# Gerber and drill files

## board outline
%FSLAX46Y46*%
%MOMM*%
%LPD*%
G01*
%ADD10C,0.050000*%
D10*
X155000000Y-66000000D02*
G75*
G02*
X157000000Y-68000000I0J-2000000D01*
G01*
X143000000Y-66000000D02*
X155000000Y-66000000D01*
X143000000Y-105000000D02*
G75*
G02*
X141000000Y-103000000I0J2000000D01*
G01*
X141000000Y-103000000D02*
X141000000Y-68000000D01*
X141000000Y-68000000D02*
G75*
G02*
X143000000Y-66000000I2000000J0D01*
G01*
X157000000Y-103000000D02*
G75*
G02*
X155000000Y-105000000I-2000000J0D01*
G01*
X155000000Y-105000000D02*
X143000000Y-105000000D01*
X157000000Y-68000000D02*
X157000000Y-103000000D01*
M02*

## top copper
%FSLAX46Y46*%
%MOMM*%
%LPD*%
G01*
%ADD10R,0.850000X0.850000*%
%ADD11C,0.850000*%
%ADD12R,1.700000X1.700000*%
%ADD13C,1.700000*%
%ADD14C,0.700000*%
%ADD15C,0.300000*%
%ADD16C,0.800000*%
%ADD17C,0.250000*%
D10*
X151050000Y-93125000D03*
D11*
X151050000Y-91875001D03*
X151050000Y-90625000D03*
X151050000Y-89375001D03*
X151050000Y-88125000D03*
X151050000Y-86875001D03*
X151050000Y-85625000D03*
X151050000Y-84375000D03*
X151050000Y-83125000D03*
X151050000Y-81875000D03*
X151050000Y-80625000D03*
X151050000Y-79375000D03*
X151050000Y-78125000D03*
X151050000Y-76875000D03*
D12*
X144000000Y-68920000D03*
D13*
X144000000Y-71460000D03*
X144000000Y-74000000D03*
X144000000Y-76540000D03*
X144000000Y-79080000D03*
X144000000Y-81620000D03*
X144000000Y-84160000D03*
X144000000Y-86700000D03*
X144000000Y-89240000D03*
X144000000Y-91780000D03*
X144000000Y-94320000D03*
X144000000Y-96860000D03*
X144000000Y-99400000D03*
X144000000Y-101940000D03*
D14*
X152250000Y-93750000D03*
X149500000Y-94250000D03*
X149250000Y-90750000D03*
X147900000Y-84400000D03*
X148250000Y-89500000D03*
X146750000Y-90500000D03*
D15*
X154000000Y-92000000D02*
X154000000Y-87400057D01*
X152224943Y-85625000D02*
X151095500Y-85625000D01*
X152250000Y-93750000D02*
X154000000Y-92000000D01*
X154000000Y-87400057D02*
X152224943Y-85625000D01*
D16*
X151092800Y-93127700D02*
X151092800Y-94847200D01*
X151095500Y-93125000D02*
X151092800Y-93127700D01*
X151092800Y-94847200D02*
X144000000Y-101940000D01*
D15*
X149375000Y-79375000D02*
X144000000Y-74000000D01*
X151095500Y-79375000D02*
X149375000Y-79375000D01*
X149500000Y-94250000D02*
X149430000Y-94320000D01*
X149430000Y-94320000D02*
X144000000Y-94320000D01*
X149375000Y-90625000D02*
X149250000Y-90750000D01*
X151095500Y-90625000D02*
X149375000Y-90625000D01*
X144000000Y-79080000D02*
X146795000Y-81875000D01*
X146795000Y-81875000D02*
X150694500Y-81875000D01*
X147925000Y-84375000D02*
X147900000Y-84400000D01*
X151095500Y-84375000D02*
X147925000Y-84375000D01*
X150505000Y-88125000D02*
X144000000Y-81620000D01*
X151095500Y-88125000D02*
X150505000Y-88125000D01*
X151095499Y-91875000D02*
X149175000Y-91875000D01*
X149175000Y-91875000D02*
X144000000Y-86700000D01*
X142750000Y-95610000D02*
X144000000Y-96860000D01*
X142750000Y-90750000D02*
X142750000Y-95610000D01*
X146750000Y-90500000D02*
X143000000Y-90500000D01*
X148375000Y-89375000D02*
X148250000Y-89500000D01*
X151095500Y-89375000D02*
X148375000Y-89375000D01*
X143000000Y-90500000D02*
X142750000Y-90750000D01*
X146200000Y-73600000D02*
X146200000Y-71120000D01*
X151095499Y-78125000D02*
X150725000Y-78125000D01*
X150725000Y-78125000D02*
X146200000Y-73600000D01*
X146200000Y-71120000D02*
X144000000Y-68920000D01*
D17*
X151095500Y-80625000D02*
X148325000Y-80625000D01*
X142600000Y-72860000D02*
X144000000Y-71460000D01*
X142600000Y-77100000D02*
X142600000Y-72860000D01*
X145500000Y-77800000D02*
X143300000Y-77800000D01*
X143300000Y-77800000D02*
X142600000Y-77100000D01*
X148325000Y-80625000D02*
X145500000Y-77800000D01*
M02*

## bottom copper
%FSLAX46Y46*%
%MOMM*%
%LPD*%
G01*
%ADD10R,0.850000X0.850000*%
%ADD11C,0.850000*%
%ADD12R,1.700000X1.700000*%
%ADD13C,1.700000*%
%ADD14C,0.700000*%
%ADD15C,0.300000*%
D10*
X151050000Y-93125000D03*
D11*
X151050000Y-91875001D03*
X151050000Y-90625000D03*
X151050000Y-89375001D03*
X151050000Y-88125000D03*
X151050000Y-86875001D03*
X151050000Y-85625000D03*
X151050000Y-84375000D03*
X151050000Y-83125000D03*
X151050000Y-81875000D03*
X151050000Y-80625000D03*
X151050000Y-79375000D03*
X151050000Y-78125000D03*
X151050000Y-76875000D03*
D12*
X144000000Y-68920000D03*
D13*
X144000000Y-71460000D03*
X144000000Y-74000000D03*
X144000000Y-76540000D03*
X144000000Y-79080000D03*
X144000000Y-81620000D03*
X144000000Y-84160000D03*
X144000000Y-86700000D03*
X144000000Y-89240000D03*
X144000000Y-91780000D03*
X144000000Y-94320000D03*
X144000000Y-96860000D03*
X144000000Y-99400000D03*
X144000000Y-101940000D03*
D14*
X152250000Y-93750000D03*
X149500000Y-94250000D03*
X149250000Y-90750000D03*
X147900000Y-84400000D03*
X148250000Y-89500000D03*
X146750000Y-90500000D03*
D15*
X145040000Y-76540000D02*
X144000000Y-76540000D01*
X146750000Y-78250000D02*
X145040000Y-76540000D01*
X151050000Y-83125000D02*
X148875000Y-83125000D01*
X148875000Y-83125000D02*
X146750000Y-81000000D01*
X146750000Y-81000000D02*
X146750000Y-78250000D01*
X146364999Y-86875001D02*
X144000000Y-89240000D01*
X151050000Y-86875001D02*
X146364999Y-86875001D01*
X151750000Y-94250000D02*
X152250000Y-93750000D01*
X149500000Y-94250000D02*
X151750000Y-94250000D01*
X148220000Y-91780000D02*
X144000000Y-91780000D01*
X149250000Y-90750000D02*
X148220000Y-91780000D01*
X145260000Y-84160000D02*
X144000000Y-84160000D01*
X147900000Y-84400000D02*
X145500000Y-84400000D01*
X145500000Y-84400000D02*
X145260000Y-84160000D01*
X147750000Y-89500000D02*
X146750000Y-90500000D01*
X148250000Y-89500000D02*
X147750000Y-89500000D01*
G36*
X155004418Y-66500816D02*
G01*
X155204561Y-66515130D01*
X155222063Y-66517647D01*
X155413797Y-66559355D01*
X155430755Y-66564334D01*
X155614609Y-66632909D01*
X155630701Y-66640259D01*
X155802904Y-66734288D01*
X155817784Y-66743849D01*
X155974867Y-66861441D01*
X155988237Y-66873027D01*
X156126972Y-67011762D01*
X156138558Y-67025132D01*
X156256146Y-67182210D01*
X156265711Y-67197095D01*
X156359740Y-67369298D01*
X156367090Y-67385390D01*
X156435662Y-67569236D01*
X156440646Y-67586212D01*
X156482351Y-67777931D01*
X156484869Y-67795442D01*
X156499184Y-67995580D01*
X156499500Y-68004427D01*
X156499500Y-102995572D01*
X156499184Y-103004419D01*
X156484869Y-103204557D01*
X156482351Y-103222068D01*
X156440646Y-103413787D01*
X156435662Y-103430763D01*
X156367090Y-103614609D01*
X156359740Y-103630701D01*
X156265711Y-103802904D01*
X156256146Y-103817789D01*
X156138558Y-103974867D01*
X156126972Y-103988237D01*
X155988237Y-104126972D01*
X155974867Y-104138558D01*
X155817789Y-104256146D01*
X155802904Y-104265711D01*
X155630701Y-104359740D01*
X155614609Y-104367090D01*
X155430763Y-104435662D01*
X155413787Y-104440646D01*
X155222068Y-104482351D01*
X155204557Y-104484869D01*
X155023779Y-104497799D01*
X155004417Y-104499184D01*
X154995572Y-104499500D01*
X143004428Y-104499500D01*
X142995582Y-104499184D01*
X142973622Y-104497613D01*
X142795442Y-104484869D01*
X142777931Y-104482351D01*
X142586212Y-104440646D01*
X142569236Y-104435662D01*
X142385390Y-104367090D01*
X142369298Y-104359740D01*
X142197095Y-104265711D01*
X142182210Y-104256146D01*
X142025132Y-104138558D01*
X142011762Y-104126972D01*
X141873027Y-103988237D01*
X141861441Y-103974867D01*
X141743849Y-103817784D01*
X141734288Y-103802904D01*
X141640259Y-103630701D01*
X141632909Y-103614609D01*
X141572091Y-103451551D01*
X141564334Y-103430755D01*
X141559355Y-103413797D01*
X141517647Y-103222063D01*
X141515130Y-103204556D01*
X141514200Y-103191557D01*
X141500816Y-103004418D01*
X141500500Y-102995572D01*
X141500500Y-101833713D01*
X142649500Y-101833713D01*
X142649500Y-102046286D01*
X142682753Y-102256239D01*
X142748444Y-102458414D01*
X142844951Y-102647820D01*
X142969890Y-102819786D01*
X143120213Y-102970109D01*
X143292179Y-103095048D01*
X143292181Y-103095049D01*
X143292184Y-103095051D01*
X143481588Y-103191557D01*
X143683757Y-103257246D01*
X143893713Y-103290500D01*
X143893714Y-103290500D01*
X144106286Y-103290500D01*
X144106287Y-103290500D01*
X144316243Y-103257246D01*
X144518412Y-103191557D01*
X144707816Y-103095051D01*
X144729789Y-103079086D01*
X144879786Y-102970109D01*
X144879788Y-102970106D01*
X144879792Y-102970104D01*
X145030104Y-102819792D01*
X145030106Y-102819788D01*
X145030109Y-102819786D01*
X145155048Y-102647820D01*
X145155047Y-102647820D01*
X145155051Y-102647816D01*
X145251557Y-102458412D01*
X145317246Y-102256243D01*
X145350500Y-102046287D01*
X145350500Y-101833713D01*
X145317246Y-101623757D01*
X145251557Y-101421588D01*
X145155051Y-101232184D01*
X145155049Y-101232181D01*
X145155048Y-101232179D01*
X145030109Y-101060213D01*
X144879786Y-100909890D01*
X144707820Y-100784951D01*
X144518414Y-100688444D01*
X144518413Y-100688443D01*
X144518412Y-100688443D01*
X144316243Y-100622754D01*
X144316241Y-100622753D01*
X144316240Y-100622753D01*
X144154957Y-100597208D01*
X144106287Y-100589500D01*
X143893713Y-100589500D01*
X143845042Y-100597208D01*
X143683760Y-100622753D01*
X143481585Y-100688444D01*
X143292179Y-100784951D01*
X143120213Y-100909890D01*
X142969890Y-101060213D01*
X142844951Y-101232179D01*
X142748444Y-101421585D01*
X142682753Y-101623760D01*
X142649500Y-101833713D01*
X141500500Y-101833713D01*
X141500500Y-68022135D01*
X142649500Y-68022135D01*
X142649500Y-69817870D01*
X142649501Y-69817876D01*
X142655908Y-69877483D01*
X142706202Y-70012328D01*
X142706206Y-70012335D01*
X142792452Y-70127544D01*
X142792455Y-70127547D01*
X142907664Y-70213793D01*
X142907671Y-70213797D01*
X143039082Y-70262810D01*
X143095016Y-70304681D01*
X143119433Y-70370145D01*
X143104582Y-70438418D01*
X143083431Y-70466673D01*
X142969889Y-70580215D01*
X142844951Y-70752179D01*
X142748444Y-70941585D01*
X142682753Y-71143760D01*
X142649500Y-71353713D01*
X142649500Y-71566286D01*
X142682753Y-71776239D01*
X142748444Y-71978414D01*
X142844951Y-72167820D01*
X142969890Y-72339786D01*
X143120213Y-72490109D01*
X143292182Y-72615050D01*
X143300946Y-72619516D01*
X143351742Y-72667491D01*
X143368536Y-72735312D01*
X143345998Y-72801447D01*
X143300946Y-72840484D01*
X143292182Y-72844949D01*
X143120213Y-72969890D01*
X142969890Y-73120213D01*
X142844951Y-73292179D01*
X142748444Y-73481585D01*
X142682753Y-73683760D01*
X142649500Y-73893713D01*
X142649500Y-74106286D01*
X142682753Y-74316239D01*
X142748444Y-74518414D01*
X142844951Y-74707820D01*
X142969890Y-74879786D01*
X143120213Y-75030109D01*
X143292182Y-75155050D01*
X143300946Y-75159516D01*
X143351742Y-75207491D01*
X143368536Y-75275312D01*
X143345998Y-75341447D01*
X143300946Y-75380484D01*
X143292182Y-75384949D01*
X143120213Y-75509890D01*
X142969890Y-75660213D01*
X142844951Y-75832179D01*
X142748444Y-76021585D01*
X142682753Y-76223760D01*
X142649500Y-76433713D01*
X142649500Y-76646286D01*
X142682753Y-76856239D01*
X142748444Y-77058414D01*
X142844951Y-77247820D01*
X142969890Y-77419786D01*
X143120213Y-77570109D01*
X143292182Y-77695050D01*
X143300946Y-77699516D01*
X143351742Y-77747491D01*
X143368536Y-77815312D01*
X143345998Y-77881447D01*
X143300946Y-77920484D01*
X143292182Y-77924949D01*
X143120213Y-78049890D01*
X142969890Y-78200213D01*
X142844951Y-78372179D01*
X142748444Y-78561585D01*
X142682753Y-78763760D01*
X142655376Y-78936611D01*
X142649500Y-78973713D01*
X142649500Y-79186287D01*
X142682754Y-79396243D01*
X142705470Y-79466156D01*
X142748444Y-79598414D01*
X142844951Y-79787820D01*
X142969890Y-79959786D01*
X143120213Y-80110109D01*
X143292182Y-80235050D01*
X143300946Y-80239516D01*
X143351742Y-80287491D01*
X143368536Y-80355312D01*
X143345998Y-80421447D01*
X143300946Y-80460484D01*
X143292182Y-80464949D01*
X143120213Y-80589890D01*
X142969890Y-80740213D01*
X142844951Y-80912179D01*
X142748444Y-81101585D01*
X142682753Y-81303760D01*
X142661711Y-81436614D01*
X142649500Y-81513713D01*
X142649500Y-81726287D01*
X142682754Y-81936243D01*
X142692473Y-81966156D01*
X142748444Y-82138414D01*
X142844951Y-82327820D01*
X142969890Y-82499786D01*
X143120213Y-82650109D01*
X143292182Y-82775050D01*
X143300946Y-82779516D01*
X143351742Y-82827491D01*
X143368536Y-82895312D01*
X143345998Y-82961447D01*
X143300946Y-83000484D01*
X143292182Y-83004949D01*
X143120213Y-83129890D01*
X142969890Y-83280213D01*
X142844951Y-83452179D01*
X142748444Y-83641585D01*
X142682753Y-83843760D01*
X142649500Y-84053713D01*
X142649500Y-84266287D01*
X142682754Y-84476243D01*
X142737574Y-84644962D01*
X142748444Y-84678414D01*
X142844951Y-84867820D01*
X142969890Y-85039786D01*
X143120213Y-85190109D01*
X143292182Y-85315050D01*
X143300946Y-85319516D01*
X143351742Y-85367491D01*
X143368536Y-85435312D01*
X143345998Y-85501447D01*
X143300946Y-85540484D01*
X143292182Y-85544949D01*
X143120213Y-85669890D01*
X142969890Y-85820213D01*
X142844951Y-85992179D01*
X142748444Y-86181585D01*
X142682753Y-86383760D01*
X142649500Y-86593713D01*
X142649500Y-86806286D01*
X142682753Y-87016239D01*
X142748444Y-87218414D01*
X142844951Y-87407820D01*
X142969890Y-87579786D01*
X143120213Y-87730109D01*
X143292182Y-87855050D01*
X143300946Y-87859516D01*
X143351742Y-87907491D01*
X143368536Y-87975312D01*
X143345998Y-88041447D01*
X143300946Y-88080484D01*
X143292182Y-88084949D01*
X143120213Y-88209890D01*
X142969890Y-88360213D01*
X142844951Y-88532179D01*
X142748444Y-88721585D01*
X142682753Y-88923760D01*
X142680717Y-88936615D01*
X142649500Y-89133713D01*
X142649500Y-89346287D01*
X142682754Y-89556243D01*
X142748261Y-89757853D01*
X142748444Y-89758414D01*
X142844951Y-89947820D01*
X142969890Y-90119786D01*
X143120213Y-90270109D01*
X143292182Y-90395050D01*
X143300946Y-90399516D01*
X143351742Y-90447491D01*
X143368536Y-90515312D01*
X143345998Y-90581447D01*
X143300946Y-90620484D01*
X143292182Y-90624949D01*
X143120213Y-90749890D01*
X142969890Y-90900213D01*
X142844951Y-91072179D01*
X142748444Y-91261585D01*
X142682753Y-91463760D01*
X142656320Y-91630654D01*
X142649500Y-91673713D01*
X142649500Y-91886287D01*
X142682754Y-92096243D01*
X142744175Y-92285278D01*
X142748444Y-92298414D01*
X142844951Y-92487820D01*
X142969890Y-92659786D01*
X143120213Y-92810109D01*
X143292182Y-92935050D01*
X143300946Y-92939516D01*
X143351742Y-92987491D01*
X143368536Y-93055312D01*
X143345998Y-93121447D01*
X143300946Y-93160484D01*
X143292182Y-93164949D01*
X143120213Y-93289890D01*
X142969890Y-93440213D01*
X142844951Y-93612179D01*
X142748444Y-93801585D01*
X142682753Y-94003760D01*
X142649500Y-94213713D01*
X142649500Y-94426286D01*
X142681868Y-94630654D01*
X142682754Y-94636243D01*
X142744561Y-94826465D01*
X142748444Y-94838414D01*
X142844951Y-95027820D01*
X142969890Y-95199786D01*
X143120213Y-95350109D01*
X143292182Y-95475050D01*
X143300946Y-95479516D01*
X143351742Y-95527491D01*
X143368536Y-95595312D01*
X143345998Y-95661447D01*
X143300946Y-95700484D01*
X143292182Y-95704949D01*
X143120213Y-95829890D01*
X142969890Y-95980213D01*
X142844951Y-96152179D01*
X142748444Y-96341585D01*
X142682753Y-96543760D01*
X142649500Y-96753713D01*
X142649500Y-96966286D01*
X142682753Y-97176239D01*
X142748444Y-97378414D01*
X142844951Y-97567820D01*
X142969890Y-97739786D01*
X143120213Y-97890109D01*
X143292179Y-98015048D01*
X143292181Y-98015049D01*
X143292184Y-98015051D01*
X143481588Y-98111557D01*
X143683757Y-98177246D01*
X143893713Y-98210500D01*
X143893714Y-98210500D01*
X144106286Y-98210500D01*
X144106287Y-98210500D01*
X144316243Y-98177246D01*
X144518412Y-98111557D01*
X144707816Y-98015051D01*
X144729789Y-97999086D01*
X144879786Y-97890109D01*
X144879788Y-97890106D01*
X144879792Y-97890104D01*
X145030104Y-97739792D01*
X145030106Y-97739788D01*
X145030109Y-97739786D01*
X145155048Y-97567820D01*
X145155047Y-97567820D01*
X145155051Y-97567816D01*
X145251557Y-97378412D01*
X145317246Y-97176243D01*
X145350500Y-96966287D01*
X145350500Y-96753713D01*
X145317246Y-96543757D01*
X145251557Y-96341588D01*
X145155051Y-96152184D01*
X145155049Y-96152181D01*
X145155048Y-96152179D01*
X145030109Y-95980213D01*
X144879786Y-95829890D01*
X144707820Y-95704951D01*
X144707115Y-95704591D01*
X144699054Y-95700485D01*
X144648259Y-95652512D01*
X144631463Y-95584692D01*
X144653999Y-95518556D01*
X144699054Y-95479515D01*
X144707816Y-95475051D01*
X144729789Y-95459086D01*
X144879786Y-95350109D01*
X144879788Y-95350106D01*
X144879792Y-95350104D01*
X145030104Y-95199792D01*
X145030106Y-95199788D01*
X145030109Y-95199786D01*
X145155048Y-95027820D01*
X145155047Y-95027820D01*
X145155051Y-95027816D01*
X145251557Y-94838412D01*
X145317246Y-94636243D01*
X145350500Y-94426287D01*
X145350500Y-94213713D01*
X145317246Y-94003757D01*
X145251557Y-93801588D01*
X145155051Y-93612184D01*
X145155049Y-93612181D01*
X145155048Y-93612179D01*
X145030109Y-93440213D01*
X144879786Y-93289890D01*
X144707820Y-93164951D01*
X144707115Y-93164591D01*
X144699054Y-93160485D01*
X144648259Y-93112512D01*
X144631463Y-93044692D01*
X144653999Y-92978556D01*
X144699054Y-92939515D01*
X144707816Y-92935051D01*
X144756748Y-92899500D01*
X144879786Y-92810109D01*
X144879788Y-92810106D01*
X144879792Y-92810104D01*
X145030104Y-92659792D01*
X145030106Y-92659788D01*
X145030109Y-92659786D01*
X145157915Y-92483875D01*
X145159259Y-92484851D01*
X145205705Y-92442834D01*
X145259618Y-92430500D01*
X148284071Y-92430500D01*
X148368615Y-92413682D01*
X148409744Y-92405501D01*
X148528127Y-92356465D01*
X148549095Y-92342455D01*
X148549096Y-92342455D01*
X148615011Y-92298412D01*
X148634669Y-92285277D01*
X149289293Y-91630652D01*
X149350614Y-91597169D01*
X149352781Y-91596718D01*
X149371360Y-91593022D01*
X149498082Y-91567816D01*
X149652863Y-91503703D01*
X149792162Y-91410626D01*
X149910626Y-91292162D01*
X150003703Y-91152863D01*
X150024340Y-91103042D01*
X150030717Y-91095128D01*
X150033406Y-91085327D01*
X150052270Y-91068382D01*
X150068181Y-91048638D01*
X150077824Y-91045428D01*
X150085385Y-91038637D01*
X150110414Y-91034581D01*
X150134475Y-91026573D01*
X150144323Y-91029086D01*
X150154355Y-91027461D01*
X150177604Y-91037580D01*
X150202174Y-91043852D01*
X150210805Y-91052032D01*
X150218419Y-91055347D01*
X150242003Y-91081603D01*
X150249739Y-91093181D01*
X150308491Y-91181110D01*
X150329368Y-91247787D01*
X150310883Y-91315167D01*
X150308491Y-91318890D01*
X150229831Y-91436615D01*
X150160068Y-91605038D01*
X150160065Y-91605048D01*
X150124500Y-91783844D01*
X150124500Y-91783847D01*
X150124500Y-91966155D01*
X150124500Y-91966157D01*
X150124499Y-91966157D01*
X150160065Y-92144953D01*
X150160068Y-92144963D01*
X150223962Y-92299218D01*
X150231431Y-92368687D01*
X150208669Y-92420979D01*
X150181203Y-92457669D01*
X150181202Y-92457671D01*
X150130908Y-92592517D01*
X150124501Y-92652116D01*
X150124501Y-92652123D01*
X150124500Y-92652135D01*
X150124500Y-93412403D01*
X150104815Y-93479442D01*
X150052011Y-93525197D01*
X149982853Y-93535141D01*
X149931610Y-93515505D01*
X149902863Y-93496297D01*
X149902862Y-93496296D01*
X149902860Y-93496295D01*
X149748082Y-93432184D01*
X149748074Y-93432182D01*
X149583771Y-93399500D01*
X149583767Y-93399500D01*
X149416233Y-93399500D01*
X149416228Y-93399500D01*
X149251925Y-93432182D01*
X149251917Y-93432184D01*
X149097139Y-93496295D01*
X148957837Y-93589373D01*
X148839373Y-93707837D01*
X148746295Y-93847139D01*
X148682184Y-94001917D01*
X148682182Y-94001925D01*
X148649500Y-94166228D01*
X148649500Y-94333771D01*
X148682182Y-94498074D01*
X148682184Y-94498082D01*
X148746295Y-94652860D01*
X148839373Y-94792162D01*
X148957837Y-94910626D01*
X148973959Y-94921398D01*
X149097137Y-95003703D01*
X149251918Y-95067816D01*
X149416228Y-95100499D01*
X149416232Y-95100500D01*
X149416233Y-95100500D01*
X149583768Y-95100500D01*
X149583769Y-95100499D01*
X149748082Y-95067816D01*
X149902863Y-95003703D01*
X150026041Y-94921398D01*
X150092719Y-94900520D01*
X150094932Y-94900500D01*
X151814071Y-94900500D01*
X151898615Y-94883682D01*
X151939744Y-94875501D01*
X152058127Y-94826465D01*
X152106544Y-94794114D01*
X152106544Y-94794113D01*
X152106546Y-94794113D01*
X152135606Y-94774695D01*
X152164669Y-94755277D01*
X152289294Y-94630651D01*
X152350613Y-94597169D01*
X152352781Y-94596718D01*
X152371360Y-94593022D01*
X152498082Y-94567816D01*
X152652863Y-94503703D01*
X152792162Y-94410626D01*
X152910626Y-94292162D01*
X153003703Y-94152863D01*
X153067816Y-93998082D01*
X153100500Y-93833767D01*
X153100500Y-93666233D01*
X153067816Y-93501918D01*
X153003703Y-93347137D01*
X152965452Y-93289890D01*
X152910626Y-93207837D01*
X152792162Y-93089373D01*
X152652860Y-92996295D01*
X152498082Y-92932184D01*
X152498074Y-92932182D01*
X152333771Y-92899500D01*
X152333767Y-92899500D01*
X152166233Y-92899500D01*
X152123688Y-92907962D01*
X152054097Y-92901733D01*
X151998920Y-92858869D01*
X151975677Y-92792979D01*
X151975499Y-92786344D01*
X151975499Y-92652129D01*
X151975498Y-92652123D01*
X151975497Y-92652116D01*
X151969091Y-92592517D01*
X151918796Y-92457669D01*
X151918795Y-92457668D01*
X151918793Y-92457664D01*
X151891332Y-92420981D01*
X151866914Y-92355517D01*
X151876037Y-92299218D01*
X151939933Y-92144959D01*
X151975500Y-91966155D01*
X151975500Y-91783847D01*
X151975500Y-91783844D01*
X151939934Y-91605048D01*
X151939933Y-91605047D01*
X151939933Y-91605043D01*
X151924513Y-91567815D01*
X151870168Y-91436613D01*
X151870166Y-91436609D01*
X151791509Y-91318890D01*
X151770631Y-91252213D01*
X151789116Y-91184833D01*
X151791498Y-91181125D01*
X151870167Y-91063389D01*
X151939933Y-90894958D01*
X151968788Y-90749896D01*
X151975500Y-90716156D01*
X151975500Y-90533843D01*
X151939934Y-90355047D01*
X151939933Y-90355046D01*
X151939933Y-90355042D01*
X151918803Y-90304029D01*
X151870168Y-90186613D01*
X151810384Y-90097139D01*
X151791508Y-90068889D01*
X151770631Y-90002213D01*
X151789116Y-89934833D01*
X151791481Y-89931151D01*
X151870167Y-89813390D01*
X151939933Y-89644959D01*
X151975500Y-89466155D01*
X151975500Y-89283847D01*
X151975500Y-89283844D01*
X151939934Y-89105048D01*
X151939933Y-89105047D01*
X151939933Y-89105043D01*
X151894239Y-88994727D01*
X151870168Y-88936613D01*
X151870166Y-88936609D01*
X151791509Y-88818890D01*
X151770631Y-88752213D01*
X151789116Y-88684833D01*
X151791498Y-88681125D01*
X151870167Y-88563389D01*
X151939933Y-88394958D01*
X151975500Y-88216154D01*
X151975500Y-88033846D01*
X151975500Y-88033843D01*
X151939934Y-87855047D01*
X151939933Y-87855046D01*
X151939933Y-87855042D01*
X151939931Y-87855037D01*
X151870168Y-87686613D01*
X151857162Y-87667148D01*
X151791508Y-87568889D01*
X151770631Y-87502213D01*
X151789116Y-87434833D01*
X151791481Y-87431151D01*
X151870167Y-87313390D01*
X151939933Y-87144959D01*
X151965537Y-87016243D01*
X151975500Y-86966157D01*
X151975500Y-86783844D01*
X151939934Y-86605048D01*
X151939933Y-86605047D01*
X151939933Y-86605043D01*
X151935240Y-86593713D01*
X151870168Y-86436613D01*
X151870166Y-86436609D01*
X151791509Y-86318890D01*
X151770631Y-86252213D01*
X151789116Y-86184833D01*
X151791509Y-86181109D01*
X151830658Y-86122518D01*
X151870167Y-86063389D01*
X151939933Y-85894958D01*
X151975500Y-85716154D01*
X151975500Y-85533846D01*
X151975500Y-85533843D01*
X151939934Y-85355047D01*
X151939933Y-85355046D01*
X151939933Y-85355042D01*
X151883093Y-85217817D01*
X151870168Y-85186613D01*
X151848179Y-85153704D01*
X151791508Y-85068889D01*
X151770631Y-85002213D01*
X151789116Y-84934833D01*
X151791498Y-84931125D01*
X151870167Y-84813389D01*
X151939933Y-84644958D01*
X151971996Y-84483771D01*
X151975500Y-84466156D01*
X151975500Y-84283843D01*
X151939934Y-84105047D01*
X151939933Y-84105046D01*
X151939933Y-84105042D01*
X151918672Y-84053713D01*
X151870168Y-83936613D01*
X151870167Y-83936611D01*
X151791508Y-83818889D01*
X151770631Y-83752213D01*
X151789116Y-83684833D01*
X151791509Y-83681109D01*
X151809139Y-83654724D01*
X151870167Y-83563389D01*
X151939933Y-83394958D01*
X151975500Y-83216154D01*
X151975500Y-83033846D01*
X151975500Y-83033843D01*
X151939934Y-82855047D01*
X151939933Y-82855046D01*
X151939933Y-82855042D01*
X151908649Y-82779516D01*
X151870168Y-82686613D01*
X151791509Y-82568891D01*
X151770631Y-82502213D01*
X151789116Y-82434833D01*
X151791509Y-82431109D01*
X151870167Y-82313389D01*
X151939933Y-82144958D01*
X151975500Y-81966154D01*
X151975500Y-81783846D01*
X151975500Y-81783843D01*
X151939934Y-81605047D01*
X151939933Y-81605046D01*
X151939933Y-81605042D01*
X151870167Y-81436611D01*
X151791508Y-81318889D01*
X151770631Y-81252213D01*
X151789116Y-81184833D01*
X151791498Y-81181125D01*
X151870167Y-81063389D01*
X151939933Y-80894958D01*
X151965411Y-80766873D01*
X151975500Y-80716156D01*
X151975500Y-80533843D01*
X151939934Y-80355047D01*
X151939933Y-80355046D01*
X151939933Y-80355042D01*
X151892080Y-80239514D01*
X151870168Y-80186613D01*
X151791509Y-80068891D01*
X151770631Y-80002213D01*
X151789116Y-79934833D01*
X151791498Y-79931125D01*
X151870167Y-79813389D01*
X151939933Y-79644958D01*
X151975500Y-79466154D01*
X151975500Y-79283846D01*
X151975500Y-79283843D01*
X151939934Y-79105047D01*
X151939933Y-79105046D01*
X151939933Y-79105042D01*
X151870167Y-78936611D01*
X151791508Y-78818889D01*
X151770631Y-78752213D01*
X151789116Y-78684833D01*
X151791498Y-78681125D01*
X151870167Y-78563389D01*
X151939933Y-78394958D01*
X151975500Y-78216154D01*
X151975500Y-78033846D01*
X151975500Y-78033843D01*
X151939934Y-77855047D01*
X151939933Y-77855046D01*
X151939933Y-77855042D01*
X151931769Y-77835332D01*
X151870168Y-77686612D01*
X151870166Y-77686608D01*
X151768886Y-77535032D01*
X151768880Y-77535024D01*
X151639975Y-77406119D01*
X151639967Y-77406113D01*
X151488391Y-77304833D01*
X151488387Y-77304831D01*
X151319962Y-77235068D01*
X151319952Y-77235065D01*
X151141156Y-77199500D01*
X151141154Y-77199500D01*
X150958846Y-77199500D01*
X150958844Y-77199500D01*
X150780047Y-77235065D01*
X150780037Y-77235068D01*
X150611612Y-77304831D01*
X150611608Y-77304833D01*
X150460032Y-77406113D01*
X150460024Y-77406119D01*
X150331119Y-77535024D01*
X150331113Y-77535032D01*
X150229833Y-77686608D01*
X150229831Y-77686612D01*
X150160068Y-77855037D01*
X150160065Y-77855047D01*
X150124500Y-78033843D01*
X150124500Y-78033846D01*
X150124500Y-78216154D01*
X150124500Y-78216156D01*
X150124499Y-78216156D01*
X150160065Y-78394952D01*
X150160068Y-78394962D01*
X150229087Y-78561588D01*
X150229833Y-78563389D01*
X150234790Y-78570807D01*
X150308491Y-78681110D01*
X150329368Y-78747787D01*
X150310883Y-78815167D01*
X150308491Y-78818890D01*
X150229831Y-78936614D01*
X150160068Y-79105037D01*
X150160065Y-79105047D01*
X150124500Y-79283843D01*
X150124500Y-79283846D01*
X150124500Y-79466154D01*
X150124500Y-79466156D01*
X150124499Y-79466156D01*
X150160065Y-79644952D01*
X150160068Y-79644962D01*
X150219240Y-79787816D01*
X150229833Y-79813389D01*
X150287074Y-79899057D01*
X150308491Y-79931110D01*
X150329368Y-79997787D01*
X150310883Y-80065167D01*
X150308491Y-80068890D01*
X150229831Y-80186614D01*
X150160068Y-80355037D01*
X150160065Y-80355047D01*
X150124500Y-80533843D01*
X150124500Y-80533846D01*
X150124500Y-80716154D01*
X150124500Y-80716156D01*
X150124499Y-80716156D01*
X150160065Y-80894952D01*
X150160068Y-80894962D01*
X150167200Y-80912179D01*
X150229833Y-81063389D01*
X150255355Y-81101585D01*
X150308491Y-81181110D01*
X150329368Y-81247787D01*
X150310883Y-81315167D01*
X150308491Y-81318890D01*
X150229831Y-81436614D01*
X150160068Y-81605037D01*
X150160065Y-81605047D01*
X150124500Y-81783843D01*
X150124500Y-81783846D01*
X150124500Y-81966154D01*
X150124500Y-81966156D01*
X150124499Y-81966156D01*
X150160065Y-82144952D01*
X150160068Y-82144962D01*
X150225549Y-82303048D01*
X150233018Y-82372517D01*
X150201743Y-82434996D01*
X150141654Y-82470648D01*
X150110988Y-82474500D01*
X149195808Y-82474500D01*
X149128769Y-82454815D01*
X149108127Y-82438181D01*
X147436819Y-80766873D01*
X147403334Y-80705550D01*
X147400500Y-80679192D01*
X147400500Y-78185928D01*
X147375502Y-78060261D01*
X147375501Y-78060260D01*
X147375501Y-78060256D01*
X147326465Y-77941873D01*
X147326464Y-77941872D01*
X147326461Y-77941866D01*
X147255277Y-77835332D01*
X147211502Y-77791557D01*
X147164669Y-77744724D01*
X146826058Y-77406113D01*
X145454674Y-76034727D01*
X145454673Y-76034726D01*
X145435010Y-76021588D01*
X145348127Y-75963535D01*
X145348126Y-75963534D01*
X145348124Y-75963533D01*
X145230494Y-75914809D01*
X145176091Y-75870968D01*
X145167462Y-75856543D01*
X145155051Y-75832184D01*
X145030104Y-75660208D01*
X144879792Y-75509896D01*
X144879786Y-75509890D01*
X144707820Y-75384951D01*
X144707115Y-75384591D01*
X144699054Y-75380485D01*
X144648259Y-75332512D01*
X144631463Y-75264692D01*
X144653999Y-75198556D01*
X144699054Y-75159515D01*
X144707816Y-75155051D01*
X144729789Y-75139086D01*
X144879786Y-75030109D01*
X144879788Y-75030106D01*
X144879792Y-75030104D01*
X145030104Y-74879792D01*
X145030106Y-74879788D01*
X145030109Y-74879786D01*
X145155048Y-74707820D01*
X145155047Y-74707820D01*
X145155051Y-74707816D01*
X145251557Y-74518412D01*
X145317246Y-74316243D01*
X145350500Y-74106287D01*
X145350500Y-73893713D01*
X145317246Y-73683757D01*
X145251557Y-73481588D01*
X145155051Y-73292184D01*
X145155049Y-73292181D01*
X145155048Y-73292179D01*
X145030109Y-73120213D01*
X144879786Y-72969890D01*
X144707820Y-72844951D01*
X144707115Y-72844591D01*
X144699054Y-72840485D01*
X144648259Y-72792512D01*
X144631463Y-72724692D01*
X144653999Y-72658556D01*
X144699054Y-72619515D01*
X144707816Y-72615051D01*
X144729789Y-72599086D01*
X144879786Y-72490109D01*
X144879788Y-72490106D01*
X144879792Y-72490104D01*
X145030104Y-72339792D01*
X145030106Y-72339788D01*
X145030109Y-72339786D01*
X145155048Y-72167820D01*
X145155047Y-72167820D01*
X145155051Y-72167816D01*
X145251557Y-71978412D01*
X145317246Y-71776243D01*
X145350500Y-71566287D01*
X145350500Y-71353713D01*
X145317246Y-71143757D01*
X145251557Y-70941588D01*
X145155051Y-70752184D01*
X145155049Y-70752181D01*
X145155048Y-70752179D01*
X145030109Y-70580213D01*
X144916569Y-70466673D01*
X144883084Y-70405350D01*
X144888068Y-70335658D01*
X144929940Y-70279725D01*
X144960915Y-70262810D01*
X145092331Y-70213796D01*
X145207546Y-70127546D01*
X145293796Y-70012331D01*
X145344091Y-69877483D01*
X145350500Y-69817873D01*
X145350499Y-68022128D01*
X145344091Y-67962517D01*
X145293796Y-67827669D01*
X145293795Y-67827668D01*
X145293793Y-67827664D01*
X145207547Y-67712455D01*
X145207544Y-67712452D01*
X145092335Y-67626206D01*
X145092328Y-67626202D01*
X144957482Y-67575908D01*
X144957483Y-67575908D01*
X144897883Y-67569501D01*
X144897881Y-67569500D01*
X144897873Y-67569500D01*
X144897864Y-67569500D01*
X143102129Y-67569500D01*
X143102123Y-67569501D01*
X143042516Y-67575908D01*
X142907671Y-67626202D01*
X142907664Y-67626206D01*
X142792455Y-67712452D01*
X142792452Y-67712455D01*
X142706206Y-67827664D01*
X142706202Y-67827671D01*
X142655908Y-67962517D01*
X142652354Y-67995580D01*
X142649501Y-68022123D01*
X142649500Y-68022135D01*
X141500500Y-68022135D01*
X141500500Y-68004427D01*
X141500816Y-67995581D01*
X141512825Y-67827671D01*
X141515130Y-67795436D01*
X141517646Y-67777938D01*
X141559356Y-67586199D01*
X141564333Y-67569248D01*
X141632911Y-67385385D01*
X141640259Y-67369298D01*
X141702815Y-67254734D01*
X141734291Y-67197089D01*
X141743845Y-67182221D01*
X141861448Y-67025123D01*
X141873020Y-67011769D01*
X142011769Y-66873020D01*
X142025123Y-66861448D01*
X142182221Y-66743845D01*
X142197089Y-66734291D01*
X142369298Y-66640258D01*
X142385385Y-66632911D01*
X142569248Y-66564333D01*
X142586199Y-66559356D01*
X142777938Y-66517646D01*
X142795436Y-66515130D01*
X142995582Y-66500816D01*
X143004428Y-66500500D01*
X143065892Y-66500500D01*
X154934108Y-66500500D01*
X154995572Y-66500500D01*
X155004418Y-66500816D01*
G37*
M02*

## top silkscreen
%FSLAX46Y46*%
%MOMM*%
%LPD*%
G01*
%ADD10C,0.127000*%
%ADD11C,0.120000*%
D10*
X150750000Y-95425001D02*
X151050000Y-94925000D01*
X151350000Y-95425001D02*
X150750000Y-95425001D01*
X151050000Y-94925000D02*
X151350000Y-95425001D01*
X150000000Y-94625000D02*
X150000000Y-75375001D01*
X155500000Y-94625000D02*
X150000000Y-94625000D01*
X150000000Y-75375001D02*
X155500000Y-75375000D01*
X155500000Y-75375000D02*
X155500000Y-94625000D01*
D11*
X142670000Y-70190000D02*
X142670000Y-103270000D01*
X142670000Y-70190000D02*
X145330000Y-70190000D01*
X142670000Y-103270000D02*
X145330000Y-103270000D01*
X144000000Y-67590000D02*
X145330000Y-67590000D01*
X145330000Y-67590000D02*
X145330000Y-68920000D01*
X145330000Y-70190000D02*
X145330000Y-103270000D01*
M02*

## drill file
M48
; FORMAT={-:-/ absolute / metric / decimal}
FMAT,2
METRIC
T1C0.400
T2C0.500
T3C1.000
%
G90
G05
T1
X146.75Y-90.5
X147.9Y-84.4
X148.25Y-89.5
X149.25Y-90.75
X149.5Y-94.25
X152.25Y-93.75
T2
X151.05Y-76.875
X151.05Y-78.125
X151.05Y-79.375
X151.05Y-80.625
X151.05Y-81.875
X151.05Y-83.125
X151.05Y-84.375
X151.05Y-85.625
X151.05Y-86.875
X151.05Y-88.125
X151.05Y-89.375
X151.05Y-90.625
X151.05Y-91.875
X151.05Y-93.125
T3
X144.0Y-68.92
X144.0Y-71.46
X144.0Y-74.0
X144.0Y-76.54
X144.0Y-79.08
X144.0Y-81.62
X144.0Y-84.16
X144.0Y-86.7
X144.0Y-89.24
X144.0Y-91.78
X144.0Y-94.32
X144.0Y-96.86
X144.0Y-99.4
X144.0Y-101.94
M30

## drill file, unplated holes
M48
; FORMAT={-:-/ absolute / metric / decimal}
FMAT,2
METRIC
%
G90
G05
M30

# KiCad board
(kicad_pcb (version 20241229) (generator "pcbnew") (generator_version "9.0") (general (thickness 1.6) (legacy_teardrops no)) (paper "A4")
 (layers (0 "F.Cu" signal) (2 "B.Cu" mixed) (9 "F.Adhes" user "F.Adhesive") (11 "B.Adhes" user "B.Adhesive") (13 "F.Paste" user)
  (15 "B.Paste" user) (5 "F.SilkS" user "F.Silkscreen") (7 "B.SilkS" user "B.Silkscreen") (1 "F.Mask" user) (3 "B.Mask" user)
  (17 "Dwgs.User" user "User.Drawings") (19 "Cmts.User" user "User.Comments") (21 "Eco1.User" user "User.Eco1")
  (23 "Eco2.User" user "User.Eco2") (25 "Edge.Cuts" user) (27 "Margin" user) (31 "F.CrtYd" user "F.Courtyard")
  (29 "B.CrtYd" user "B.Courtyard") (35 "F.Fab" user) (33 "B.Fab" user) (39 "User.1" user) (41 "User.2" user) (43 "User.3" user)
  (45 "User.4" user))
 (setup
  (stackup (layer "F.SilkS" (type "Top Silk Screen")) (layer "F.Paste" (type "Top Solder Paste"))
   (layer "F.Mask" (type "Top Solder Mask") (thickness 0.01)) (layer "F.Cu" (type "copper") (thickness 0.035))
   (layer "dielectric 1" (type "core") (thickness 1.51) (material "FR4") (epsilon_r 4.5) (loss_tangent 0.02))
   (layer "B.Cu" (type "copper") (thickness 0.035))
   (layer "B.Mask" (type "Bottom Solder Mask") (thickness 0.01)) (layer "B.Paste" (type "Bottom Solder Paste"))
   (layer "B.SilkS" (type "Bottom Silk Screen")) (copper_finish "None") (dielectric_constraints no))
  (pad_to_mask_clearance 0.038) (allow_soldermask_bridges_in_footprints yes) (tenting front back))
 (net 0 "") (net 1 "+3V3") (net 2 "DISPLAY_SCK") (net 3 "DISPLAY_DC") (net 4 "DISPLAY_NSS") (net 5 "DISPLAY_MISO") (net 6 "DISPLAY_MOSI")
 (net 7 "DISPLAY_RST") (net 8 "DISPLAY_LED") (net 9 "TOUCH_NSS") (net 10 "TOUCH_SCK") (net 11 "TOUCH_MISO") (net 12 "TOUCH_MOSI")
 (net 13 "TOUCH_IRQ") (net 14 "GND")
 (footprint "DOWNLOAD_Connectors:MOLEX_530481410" (layer "F.Cu") (at 151.05 93.125 90)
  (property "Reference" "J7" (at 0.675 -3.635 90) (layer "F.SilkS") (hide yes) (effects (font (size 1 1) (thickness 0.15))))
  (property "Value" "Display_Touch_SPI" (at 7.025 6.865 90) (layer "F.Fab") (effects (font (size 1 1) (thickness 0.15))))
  (fp_line (start 17.749999 -1.05) (end 17.75 4.45) (stroke (width 0.127) (type solid)) (layer "F.SilkS"))
  (fp_line (start -1.5 -1.05) (end 17.749999 -1.05) (stroke (width 0.127) (type solid)) (layer "F.SilkS"))
  (fp_line (start -2.300001 -0.3) (end -1.8 0) (stroke (width 0.127) (type solid)) (layer "F.SilkS"))
  (fp_line (start -1.8 0) (end -2.300001 0.3) (stroke (width 0.127) (type solid)) (layer "F.SilkS"))
  (fp_line (start -2.300001 0.3) (end -2.300001 -0.3) (stroke (width 0.127) (type solid)) (layer "F.SilkS"))
  (fp_line (start 17.75 4.45) (end -1.5 4.45) (stroke (width 0.127) (type solid)) (layer "F.SilkS"))
  (fp_line (start -1.5 4.45) (end -1.5 -1.05) (stroke (width 0.127) (type solid)) (layer "F.SilkS"))
  (pad "1" thru_hole rect (at 0 0 90) (size 0.85 0.85) (drill 0.5) (layers "*.Cu") (remove_unused_layers no) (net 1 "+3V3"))
  (pad "2" thru_hole circle (at 1.249999 0 90) (size 0.85 0.85) (drill 0.5) (layers "*.Cu") (remove_unused_layers no) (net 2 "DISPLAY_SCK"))
  (pad "3" thru_hole circle (at 2.5 0 90) (size 0.85 0.85) (drill 0.5) (layers "*.Cu") (remove_unused_layers no) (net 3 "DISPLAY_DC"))
  (pad "4" thru_hole circle (at 3.749999 0 90) (size 0.85 0.85) (drill 0.5) (layers "*.Cu") (remove_unused_layers no) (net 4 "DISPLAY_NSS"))
  (pad "5" thru_hole circle (at 5 0 90) (size 0.85 0.85) (drill 0.5) (layers "*.Cu") (remove_unused_layers no) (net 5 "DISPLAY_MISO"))
  (pad "6" thru_hole circle (at 6.249999 0 90) (size 0.85 0.85) (drill 0.5) (layers "*.Cu") (remove_unused_layers no) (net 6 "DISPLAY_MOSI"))
  (pad "7" thru_hole circle (at 7.5 0 90) (size 0.85 0.85) (drill 0.5) (layers "*.Cu") (remove_unused_layers no) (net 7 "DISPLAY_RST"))
  (pad "8" thru_hole circle (at 8.75 0 90) (size 0.85 0.85) (drill 0.5) (layers "*.Cu") (remove_unused_layers no) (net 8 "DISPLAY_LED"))
  (pad "9" thru_hole circle (at 10 0 90) (size 0.85 0.85) (drill 0.5) (layers "*.Cu") (remove_unused_layers no) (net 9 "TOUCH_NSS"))
  (pad "10" thru_hole circle (at 11.25 0 90) (size 0.85 0.85) (drill 0.5) (layers "*.Cu") (remove_unused_layers no) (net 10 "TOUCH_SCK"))
  (pad "11" thru_hole circle (at 12.5 0 90) (size 0.85 0.85) (drill 0.5) (layers "*.Cu") (remove_unused_layers no) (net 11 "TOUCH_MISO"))
  (pad "12" thru_hole circle (at 13.75 0 90) (size 0.85 0.85) (drill 0.5) (layers "*.Cu") (remove_unused_layers no) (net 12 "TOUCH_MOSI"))
  (pad "13" thru_hole circle (at 15 0 90) (size 0.85 0.85) (drill 0.5) (layers "*.Cu") (remove_unused_layers no) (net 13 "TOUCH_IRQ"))
  (pad "14" thru_hole circle (at 16.25 0 90) (size 0.85 0.85) (drill 0.5) (layers "*.Cu") (remove_unused_layers no) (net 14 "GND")))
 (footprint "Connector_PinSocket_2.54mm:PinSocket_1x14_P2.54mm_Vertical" (layer "F.Cu") (at 144 68.92)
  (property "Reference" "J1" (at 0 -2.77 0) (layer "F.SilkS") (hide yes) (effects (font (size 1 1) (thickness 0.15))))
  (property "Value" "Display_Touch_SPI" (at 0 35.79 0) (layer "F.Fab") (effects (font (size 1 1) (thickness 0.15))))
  (fp_line (start -1.33 1.27) (end -1.33 34.35) (stroke (width 0.12) (type solid)) (layer "F.SilkS"))
  (fp_line (start -1.33 1.27) (end 1.33 1.27) (stroke (width 0.12) (type solid)) (layer "F.SilkS"))
  (fp_line (start -1.33 34.35) (end 1.33 34.35) (stroke (width 0.12) (type solid)) (layer "F.SilkS"))
  (fp_line (start 0 -1.33) (end 1.33 -1.33) (stroke (width 0.12) (type solid)) (layer "F.SilkS"))
  (fp_line (start 1.33 -1.33) (end 1.33 0) (stroke (width 0.12) (type solid)) (layer "F.SilkS"))
  (fp_line (start 1.33 1.27) (end 1.33 34.35) (stroke (width 0.12) (type solid)) (layer "F.SilkS"))
  (pad "1" thru_hole rect (at 0 0) (size 1.7 1.7) (drill 1) (layers "*.Cu" "*.Mask") (remove_unused_layers no) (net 13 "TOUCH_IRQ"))
  (pad "2" thru_hole circle (at 0 2.54) (size 1.7 1.7) (drill 1) (layers "*.Cu" "*.Mask") (remove_unused_layers no) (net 11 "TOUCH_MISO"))
  (pad "3" thru_hole circle (at 0 5.08) (size 1.7 1.7) (drill 1) (layers "*.Cu" "*.Mask") (remove_unused_layers no) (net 12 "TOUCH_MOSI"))
  (pad "4" thru_hole circle (at 0 7.62) (size 1.7 1.7) (drill 1) (layers "*.Cu" "*.Mask") (remove_unused_layers no) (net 9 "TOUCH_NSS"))
  (pad "5" thru_hole circle (at 0 10.16) (size 1.7 1.7) (drill 1) (layers "*.Cu" "*.Mask") (remove_unused_layers no) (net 10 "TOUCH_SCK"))
  (pad "6" thru_hole circle (at 0 12.7) (size 1.7 1.7) (drill 1) (layers "*.Cu" "*.Mask") (remove_unused_layers no) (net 5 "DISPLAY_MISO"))
  (pad "7" thru_hole circle (at 0 15.24) (size 1.7 1.7) (drill 1) (layers "*.Cu" "*.Mask") (remove_unused_layers no) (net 8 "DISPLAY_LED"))
  (pad "8" thru_hole circle (at 0 17.78) (size 1.7 1.7) (drill 1) (layers "*.Cu" "*.Mask") (remove_unused_layers no) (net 2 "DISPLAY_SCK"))
  (pad "9" thru_hole circle (at 0 20.32) (size 1.7 1.7) (drill 1) (layers "*.Cu" "*.Mask") (remove_unused_layers no) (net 6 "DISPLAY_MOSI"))
  (pad "10" thru_hole circle (at 0 22.86) (size 1.7 1.7) (drill 1) (layers "*.Cu" "*.Mask") (remove_unused_layers no) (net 3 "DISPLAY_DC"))
  (pad "11" thru_hole circle (at 0 25.4) (size 1.7 1.7) (drill 1) (layers "*.Cu" "*.Mask") (remove_unused_layers no) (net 7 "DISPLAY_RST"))
  (pad "12" thru_hole circle (at 0 27.94) (size 1.7 1.7) (drill 1) (layers "*.Cu" "*.Mask") (remove_unused_layers no) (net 4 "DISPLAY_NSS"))
  (pad "13" thru_hole circle (at 0 30.48) (size 1.7 1.7) (drill 1) (layers "*.Cu" "*.Mask") (remove_unused_layers no) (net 14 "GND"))
  (pad "14" thru_hole circle (at 0 33.02) (size 1.7 1.7) (drill 1) (layers "*.Cu" "*.Mask") (remove_unused_layers no) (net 1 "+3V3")))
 (gr_arc (start 155 66) (mid 156.414214 66.585786) (end 157 68) (stroke (width 0.05) (type default)) (layer "Edge.Cuts"))
 (gr_line (start 143 66) (end 155 66) (stroke (width 0.05) (type default)) (layer "Edge.Cuts"))
 (gr_arc (start 143 105) (mid 141.585786 104.414214) (end 141 103) (stroke (width 0.05) (type default)) (layer "Edge.Cuts"))
 (gr_line (start 141 103) (end 141 68) (stroke (width 0.05) (type default)) (layer "Edge.Cuts"))
 (gr_arc (start 141 68) (mid 141.585786 66.585786) (end 143 66) (stroke (width 0.05) (type default)) (layer "Edge.Cuts"))
 (gr_arc (start 157 103) (mid 156.414214 104.414214) (end 155 105) (stroke (width 0.05) (type default)) (layer "Edge.Cuts"))
 (gr_line (start 155 105) (end 143 105) (stroke (width 0.05) (type default)) (layer "Edge.Cuts"))
 (gr_line (start 157 68) (end 157 103) (stroke (width 0.05) (type default)) (layer "Edge.Cuts"))
 (segment (start 151.0928 93.1277) (end 151.0928 94.8472) (width 0.8) (layer "F.Cu") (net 1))
 (segment (start 151.0955 93.125) (end 151.0928 93.1277) (width 0.8) (layer "F.Cu") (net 1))
 (segment (start 151.0928 94.8472) (end 144 101.94) (width 0.8) (layer "F.Cu") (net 1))
 (segment (start 149.375 79.375) (end 144 74) (width 0.3) (layer "F.Cu") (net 12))
 (segment (start 151.0955 79.375) (end 149.375 79.375) (width 0.3) (layer "F.Cu") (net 12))
 (segment (start 154 87.400057) (end 152.224943 85.625) (width 0.3) (layer "F.Cu") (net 7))
 (segment (start 149.5 94.25) (end 149.43 94.32) (width 0.3) (layer "F.Cu") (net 7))
 (segment (start 149.43 94.32) (end 144 94.32) (width 0.3) (layer "F.Cu") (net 7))
 (segment (start 152.224943 85.625) (end 151.0955 85.625) (width 0.3) (layer "F.Cu") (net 7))
 (segment (start 152.25 93.75) (end 154 92) (width 0.3) (layer "F.Cu") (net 7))
 (segment (start 154 92) (end 154 87.400057) (width 0.3) (layer "F.Cu") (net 7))
 (via (at 149.5 94.25) (size 0.7) (drill 0.4) (layers "F.Cu" "B.Cu") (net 7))
 (via (at 152.25 93.75) (size 0.7) (drill 0.4) (layers "F.Cu" "B.Cu") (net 7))
 (segment (start 151.75 94.25) (end 152.25 93.75) (width 0.3) (layer "B.Cu") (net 7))
 (segment (start 149.5 94.25) (end 151.75 94.25) (width 0.3) (layer "B.Cu") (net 7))
 (segment (start 149.375 90.625) (end 149.25 90.75) (width 0.3) (layer "F.Cu") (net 3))
 (segment (start 151.0955 90.625) (end 149.375 90.625) (width 0.3) (layer "F.Cu") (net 3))
 (via (at 149.25 90.75) (size 0.7) (drill 0.4) (layers "F.Cu" "B.Cu") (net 3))
 (segment (start 148.22 91.78) (end 144 91.78) (width 0.3) (layer "B.Cu") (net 3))
 (segment (start 149.25 90.75) (end 148.22 91.78) (width 0.3) (layer "B.Cu") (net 3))
 (segment (start 144 79.08) (end 146.795 81.875) (width 0.3) (layer "F.Cu") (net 10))
 (segment (start 146.795 81.875) (end 150.6945 81.875) (width 0.3) (layer "F.Cu") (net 10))
 (segment (start 146.364999 86.875001) (end 144 89.24) (width 0.3) (layer "B.Cu") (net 6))
 (segment (start 151.05 86.875001) (end 146.364999 86.875001) (width 0.3) (layer "B.Cu") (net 6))
 (segment (start 147.925 84.375) (end 147.9 84.4) (width 0.3) (layer "F.Cu") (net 8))
 (segment (start 151.0955 84.375) (end 147.925 84.375) (width 0.3) (layer "F.Cu") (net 8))
 (via (at 147.9 84.4) (size 0.7) (drill 0.4) (layers "F.Cu" "B.Cu") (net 8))
 (segment (start 145.26 84.16) (end 144 84.16) (width 0.3) (layer "B.Cu") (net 8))
 (segment (start 147.9 84.4) (end 145.5 84.4) (width 0.3) (layer "B.Cu") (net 8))
 (segment (start 145.5 84.4) (end 145.26 84.16) (width 0.3) (layer "B.Cu") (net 8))
 (segment (start 150.505 88.125) (end 144 81.62) (width 0.3) (layer "F.Cu") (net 5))
 (segment (start 151.0955 88.125) (end 150.505 88.125) (width 0.3) (layer "F.Cu") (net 5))
 (segment (start 146.75 78.25) (end 145.04 76.54) (width 0.3) (layer "B.Cu") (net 9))
 (segment (start 145.04 76.54) (end 144 76.54) (width 0.3) (layer "B.Cu") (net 9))
 (segment (start 148.875 83.125) (end 146.75 81) (width 0.3) (layer "B.Cu") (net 9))
 (segment (start 146.75 81) (end 146.75 78.25) (width 0.3) (layer "B.Cu") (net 9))
 (segment (start 151.05 83.125) (end 148.875 83.125) (width 0.3) (layer "B.Cu") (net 9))
 (segment (start 151.095499 91.875) (end 149.175 91.875) (width 0.3) (layer "F.Cu") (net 2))
 (segment (start 149.175 91.875) (end 144 86.7) (width 0.3) (layer "F.Cu") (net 2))
 (segment (start 142.75 95.61) (end 144 96.86) (width 0.3) (layer "F.Cu") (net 4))
 (segment (start 142.75 90.75) (end 142.75 95.61) (width 0.3) (layer "F.Cu") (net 4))
 (segment (start 146.75 90.5) (end 143 90.5) (width 0.3) (layer "F.Cu") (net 4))
 (segment (start 148.375 89.375) (end 148.25 89.5) (width 0.3) (layer "F.Cu") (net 4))
 (segment (start 151.0955 89.375) (end 148.375 89.375) (width 0.3) (layer "F.Cu") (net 4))
 (segment (start 143 90.5) (end 142.75 90.75) (width 0.3) (layer "F.Cu") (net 4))
 (via (at 148.25 89.5) (size 0.7) (drill 0.4) (layers "F.Cu" "B.Cu") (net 4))
 (via (at 146.75 90.5) (size 0.7) (drill 0.4) (layers "F.Cu" "B.Cu") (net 4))
 (segment (start 147.75 89.5) (end 146.75 90.5) (width 0.3) (layer "B.Cu") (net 4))
 (segment (start 148.25 89.5) (end 147.75 89.5) (width 0.3) (layer "B.Cu") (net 4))
 (segment (start 146.2 73.6) (end 146.2 71.12) (width 0.3) (layer "F.Cu") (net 13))
 (segment (start 151.095499 78.125) (end 150.725 78.125) (width 0.3) (layer "F.Cu") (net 13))
 (segment (start 150.725 78.125) (end 146.2 73.6) (width 0.3) (layer "F.Cu") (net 13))
 (segment (start 146.2 71.12) (end 144 68.92) (width 0.3) (layer "F.Cu") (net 13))
 (segment (start 151.0955 80.625) (end 148.325 80.625) (width 0.25) (layer "F.Cu") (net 11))
 (segment (start 142.6 72.86) (end 144 71.46) (width 0.25) (layer "F.Cu") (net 11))
 (segment (start 142.6 77.1) (end 142.6 72.86) (width 0.25) (layer "F.Cu") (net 11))
 (segment (start 145.5 77.8) (end 143.3 77.8) (width 0.25) (layer "F.Cu") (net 11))
 (segment (start 143.3 77.8) (end 142.6 77.1) (width 0.25) (layer "F.Cu") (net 11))
 (segment (start 148.325 80.625) (end 145.5 77.8) (width 0.25) (layer "F.Cu") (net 11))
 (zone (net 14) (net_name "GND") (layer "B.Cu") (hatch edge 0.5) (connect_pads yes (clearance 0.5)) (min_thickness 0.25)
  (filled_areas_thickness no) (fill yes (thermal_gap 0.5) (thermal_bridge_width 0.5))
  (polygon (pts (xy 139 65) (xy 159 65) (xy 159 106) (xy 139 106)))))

